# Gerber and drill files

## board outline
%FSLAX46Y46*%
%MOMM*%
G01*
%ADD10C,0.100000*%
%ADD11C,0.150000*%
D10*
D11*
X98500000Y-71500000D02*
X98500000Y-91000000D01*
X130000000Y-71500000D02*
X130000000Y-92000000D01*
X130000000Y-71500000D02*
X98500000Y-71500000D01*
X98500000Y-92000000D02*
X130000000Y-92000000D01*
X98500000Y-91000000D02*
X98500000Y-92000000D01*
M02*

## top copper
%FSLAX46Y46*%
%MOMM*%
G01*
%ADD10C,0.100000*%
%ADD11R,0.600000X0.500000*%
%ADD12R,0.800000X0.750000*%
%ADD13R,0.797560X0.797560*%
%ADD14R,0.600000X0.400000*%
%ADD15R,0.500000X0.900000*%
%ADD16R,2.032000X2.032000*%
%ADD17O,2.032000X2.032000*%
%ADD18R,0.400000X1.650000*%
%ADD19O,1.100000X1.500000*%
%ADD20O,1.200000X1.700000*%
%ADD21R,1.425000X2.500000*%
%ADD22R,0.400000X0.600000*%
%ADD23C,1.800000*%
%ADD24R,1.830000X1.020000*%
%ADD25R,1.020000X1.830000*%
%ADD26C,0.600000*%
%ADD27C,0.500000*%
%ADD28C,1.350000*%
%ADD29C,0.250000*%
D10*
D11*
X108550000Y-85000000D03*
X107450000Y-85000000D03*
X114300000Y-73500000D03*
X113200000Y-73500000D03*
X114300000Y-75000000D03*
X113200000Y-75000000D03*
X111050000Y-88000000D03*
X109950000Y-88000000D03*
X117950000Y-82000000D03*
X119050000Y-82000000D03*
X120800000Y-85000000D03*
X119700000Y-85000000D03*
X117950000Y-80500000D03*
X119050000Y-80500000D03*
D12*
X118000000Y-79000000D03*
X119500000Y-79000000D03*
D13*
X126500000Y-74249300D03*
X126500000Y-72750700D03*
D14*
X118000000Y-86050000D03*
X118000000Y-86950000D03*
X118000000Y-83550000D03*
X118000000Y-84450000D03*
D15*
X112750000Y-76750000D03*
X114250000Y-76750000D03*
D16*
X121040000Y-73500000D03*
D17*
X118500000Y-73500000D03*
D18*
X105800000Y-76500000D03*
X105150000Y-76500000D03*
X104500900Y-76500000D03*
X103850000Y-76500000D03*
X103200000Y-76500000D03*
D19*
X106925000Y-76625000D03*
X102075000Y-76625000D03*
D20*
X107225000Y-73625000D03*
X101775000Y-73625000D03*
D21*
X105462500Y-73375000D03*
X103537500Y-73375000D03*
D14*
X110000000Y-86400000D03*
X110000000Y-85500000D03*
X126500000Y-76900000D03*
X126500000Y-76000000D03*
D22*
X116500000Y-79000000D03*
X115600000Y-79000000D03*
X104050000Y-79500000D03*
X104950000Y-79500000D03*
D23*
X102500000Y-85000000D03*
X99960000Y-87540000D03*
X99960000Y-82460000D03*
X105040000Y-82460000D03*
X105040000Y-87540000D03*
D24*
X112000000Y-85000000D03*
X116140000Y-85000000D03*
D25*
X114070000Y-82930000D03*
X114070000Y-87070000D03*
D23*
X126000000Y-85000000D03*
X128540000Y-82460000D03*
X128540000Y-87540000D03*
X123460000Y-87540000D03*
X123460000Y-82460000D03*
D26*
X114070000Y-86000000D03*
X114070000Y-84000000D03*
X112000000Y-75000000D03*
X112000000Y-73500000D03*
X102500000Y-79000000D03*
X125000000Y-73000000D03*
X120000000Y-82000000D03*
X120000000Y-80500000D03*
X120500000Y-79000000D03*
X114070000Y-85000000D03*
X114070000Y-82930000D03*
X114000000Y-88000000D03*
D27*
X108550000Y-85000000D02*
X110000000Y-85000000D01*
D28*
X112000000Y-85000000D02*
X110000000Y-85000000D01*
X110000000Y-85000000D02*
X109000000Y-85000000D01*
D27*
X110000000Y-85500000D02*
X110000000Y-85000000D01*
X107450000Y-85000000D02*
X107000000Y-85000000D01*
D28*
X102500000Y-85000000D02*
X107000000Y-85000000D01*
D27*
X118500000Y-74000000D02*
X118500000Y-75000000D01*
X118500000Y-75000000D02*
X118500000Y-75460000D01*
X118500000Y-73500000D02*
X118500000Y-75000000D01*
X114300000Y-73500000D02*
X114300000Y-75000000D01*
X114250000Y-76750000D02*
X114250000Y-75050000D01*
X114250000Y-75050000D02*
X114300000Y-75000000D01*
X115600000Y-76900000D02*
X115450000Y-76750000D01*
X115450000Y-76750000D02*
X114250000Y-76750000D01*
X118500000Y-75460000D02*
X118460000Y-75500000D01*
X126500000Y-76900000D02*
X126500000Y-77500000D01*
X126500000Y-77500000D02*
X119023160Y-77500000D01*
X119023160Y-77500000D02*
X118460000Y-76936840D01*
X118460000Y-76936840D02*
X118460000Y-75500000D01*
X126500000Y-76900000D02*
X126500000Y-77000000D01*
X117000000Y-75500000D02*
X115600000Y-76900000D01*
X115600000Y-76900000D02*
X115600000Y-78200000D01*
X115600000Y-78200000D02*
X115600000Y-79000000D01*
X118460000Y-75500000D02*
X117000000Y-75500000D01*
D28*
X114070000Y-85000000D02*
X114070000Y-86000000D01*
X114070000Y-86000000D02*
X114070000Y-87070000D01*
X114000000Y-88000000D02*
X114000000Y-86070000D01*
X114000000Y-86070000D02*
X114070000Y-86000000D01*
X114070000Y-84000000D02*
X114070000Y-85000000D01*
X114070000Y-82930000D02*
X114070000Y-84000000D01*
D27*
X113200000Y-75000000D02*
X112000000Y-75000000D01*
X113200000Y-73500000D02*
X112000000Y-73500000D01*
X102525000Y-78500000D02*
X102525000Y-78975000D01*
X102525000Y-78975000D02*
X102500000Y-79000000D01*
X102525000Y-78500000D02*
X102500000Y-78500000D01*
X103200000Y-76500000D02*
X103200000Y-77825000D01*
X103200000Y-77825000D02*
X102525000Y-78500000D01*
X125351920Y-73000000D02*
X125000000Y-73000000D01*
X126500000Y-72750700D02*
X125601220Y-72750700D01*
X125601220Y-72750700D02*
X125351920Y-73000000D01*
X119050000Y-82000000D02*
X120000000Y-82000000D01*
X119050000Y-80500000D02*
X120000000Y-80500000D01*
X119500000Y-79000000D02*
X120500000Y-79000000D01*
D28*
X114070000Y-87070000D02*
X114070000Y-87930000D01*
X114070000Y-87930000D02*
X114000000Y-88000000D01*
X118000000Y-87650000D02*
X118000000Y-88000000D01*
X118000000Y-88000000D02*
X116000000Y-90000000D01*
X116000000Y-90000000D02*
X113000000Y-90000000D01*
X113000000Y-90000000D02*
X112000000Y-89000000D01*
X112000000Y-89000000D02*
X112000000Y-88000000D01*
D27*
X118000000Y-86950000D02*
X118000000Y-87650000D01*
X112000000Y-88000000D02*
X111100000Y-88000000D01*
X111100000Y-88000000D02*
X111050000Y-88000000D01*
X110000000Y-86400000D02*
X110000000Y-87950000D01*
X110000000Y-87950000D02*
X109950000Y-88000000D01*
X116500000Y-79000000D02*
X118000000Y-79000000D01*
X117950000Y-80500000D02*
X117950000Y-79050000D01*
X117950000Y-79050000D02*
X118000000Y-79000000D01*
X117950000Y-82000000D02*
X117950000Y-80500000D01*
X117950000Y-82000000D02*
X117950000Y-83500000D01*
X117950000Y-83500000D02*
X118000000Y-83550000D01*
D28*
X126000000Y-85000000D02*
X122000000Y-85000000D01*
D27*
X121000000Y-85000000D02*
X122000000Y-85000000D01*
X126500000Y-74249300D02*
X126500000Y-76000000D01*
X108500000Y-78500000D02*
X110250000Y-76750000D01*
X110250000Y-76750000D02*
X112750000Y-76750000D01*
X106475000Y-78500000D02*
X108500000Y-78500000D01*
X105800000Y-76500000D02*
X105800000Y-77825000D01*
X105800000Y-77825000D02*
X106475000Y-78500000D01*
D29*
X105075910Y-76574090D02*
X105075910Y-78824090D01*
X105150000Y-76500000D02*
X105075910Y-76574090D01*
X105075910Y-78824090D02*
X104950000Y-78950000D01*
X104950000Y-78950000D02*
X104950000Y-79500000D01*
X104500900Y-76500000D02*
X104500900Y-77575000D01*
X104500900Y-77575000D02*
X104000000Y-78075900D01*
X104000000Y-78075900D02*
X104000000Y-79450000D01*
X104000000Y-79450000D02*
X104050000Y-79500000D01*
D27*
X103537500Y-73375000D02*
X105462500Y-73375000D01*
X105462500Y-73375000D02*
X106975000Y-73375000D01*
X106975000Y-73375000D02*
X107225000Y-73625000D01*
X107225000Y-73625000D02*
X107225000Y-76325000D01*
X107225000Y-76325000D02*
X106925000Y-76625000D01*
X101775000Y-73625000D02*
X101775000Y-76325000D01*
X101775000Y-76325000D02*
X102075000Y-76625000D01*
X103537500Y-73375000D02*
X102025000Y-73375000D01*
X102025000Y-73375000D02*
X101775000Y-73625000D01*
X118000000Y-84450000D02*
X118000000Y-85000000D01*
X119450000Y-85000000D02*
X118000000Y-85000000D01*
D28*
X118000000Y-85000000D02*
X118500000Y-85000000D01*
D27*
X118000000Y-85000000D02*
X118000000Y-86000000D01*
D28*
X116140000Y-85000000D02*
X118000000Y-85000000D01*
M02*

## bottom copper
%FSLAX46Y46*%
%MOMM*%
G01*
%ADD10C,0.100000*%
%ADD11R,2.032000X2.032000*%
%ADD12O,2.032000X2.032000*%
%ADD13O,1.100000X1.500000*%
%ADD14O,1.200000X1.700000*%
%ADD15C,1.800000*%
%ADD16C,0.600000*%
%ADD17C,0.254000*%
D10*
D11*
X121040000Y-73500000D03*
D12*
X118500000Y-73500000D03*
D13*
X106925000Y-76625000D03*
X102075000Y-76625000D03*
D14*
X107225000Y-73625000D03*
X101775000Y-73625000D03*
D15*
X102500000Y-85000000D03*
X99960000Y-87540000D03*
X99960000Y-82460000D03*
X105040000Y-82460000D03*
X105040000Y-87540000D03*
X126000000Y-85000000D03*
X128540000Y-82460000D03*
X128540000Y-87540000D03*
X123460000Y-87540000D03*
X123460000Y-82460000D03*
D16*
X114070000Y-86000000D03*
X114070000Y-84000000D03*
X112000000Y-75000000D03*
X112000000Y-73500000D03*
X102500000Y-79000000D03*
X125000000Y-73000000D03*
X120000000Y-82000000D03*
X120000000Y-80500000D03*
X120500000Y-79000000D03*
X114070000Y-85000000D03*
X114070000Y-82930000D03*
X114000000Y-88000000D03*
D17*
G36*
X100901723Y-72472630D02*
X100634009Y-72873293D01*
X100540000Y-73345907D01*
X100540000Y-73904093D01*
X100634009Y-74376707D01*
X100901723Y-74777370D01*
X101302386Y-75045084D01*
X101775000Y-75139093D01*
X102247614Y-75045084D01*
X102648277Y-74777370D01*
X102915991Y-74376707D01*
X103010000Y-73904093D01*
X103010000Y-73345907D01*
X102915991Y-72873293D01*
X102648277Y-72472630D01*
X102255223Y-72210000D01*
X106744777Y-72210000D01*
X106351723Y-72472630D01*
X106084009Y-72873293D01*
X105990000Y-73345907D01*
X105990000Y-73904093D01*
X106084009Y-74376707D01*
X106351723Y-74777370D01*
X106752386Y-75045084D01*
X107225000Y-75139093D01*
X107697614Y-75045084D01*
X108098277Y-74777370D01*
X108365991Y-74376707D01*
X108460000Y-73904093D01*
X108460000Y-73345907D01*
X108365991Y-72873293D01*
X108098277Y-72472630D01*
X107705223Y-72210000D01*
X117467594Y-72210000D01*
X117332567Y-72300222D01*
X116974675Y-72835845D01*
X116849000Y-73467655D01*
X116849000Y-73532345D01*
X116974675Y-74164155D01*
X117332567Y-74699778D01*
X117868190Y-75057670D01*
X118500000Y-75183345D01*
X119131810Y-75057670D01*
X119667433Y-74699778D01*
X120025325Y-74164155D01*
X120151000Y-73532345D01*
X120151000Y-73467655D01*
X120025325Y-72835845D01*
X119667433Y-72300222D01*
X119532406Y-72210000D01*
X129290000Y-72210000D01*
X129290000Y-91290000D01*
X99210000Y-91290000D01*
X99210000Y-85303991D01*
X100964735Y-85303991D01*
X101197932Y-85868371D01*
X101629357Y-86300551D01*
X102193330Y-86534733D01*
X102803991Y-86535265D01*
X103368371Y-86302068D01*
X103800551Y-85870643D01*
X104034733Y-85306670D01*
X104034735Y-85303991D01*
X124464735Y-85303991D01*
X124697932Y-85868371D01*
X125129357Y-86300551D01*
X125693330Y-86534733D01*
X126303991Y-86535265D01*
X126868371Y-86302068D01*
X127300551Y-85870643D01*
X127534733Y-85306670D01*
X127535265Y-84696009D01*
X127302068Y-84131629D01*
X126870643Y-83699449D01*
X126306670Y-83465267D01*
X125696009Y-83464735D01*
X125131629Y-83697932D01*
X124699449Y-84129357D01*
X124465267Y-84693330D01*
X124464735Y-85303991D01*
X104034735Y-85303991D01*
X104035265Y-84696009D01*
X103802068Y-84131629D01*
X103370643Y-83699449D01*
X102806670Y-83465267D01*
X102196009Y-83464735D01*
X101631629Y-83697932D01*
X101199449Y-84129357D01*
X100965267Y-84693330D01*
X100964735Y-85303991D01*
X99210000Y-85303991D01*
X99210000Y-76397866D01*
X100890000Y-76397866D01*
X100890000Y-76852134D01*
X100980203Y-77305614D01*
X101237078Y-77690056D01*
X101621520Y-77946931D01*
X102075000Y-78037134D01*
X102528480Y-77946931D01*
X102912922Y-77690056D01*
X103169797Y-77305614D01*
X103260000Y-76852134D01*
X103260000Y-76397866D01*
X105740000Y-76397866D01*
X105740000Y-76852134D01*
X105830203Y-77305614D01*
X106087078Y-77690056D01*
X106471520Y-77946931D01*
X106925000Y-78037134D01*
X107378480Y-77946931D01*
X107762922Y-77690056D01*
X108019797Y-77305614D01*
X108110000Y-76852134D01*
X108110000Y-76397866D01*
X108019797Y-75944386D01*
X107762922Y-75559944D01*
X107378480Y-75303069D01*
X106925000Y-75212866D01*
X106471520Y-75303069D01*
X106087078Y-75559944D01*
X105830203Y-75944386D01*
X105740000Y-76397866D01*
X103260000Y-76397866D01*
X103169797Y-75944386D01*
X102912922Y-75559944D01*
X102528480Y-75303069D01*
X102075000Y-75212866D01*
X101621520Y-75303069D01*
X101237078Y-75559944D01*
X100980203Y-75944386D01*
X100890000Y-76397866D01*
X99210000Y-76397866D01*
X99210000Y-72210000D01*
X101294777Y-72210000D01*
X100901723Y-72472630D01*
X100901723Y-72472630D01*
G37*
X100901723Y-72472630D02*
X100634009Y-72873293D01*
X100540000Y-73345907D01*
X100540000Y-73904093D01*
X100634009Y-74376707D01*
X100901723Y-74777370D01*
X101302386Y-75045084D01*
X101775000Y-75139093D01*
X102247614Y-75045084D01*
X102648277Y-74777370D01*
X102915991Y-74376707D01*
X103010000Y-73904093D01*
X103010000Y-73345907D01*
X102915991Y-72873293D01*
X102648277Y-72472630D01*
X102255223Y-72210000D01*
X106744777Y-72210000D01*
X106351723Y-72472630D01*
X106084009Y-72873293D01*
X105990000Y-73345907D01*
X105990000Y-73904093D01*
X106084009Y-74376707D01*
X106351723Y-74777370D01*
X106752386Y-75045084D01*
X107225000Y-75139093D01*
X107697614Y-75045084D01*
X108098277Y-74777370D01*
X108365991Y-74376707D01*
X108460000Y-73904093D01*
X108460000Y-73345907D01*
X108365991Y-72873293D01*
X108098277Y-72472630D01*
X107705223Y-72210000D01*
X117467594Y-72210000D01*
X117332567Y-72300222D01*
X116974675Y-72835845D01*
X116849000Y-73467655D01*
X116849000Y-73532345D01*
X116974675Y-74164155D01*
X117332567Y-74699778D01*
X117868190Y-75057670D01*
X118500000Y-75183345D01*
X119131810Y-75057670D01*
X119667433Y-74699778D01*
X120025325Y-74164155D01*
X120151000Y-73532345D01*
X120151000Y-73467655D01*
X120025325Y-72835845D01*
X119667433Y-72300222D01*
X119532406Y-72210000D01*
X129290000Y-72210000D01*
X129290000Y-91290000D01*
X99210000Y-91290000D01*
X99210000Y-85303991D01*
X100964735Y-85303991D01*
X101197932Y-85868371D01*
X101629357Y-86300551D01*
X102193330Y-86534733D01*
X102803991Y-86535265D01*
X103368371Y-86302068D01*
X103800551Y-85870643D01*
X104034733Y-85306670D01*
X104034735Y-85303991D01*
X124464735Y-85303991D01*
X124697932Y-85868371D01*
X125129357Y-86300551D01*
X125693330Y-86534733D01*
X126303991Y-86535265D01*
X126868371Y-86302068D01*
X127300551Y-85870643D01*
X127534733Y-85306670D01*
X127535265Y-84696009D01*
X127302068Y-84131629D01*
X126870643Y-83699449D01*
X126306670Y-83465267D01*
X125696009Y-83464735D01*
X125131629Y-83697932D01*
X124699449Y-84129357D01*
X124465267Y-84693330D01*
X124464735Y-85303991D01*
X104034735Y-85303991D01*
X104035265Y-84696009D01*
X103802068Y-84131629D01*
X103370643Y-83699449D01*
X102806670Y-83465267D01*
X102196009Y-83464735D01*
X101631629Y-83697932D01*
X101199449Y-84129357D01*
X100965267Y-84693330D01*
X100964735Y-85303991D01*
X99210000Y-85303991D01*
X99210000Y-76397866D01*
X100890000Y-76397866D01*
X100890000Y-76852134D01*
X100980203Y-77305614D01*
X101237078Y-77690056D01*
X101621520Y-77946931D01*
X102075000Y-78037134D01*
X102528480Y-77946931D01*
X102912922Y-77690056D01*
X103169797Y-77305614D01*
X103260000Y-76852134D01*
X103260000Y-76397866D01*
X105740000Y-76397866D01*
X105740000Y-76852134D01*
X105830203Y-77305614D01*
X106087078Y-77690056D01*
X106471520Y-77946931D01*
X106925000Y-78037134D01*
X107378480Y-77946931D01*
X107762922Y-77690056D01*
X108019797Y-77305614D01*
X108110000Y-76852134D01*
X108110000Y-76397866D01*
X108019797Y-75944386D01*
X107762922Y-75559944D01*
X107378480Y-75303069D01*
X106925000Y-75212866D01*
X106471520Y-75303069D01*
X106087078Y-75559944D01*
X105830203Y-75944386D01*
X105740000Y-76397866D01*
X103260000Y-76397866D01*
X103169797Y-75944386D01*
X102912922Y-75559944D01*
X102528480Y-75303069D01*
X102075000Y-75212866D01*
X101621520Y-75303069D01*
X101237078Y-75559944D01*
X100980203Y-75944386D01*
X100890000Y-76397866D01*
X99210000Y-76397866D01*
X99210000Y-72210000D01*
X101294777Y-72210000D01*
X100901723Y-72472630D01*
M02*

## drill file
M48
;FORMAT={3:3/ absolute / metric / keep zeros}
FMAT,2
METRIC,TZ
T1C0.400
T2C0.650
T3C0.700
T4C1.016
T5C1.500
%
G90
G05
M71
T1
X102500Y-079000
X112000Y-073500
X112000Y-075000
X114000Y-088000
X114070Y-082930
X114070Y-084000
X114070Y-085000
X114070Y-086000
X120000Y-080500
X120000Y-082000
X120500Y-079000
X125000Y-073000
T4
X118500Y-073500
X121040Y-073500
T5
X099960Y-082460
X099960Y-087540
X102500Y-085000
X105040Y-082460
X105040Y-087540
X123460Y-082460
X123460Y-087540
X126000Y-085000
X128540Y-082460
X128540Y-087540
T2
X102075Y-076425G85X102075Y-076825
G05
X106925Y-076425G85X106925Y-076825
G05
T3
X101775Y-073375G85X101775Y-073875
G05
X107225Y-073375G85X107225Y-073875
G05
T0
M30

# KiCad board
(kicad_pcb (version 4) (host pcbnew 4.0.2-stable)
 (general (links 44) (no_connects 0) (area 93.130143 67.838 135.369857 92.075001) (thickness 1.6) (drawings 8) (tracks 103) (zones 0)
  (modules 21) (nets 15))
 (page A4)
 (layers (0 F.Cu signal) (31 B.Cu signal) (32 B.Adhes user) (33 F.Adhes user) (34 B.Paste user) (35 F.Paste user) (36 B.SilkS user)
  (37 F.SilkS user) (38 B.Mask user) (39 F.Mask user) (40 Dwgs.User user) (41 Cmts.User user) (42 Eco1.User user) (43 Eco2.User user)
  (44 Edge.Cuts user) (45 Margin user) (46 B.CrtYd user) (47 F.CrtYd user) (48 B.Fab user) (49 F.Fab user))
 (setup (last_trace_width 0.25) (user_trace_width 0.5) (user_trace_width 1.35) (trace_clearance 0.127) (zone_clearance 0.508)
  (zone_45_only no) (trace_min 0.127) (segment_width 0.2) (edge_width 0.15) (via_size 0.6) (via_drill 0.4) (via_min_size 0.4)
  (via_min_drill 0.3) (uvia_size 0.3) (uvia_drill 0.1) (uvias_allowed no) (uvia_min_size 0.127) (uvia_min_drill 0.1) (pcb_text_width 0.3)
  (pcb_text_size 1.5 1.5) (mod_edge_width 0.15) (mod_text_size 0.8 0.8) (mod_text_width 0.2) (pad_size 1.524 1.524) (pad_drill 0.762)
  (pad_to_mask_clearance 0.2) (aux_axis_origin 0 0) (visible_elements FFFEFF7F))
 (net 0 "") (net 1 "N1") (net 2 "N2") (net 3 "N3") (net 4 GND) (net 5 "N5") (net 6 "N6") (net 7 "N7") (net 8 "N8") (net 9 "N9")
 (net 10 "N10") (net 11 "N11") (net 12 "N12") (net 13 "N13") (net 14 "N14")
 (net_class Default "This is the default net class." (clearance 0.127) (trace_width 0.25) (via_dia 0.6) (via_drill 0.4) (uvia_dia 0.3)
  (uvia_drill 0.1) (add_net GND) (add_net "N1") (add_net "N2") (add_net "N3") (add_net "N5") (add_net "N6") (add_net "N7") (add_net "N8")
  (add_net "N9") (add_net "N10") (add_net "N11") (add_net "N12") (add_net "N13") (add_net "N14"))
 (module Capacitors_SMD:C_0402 (layer F.Cu) (at 108 85 180)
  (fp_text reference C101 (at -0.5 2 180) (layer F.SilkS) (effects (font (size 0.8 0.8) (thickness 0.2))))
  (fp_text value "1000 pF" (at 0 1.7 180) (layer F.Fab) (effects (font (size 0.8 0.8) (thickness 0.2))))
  (pad 1 smd rect (at -0.55 0 180) (size 0.6 0.5) (layers F.Cu F.Paste F.Mask) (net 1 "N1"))
  (pad 2 smd rect (at 0.55 0 180) (size 0.6 0.5) (layers F.Cu F.Paste F.Mask) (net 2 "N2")))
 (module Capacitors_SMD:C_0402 (layer F.Cu) (at 113.75 73.5 180)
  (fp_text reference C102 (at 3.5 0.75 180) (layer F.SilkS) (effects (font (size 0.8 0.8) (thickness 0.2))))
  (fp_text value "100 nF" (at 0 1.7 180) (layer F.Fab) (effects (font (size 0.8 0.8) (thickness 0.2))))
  (pad 1 smd rect (at -0.55 0 180) (size 0.6 0.5) (layers F.Cu F.Paste F.Mask) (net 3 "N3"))
  (pad 2 smd rect (at 0.55 0 180) (size 0.6 0.5) (layers F.Cu F.Paste F.Mask) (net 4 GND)))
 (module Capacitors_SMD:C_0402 (layer F.Cu) (at 113.75 75 180)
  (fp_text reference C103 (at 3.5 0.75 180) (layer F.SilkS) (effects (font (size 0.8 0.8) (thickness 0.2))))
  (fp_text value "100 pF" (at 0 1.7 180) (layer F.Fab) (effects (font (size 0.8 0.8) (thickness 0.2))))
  (pad 1 smd rect (at -0.55 0 180) (size 0.6 0.5) (layers F.Cu F.Paste F.Mask) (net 3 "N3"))
  (pad 2 smd rect (at 0.55 0 180) (size 0.6 0.5) (layers F.Cu F.Paste F.Mask) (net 4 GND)))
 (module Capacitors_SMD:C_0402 (layer F.Cu) (at 110.5 88 180)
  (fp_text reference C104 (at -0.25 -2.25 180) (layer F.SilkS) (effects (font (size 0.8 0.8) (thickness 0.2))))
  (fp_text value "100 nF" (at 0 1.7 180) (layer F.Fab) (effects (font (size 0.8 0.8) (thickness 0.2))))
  (pad 1 smd rect (at -0.55 0 180) (size 0.6 0.5) (layers F.Cu F.Paste F.Mask) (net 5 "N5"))
  (pad 2 smd rect (at 0.55 0 180) (size 0.6 0.5) (layers F.Cu F.Paste F.Mask) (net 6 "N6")))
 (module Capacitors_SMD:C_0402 (layer F.Cu) (at 118.5 82)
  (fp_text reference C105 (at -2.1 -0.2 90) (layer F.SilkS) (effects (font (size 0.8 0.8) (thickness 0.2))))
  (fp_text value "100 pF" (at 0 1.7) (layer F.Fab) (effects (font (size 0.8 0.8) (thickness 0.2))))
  (pad 1 smd rect (at -0.55 0) (size 0.6 0.5) (layers F.Cu F.Paste F.Mask) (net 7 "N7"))
  (pad 2 smd rect (at 0.55 0) (size 0.6 0.5) (layers F.Cu F.Paste F.Mask) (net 4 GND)))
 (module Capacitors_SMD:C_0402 (layer F.Cu) (at 120.25 85 180)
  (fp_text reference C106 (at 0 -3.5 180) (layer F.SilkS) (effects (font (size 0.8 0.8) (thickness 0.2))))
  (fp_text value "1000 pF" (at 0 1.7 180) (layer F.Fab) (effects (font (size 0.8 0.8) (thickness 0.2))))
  (pad 1 smd rect (at -0.55 0 180) (size 0.6 0.5) (layers F.Cu F.Paste F.Mask) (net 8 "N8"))
  (pad 2 smd rect (at 0.55 0 180) (size 0.6 0.5) (layers F.Cu F.Paste F.Mask) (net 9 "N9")))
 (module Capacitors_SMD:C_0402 (layer F.Cu) (at 118.5 80.5)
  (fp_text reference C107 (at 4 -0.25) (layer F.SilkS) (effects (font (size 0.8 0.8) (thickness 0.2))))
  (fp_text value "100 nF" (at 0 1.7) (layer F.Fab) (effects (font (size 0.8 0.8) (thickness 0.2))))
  (pad 1 smd rect (at -0.55 0) (size 0.6 0.5) (layers F.Cu F.Paste F.Mask) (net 7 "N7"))
  (pad 2 smd rect (at 0.55 0) (size 0.6 0.5) (layers F.Cu F.Paste F.Mask) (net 4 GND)))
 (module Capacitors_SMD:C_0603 (layer F.Cu) (at 118.75 79)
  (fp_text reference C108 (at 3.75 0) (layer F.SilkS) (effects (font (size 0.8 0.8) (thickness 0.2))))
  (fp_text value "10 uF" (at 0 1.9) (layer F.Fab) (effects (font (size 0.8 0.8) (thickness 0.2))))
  (pad 1 smd rect (at -0.75 0) (size 0.8 0.75) (layers F.Cu F.Paste F.Mask) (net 7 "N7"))
  (pad 2 smd rect (at 0.75 0) (size 0.8 0.75) (layers F.Cu F.Paste F.Mask) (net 4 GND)))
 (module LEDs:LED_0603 (layer F.Cu) (at 126.5 73.5 270)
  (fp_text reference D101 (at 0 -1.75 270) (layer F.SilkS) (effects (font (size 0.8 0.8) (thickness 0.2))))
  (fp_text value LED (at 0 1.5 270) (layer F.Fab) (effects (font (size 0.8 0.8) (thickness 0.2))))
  (pad 2 smd rect (at 0.7493 0 90) (size 0.79756 0.79756) (layers F.Cu F.Paste F.Mask) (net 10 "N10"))
  (pad 1 smd rect (at -0.7493 0 90) (size 0.79756 0.79756) (layers F.Cu F.Paste F.Mask) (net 4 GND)))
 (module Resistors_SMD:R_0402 (layer F.Cu) (at 118 86.5 270)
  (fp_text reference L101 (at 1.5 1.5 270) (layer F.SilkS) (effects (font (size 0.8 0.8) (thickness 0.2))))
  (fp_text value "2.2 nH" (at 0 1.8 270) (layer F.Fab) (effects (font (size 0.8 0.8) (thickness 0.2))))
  (pad 1 smd rect (at -0.45 0 270) (size 0.4 0.6) (layers F.Cu F.Paste F.Mask) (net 9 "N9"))
  (pad 2 smd rect (at 0.45 0 270) (size 0.4 0.6) (layers F.Cu F.Paste F.Mask) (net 5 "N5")))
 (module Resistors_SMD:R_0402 (layer F.Cu) (at 118 84 270)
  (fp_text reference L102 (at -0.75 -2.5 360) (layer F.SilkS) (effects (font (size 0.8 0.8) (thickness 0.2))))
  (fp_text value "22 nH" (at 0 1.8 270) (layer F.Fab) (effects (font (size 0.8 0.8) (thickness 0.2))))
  (pad 1 smd rect (at -0.45 0 270) (size 0.4 0.6) (layers F.Cu F.Paste F.Mask) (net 7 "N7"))
  (pad 2 smd rect (at 0.45 0 270) (size 0.4 0.6) (layers F.Cu F.Paste F.Mask) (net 9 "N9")))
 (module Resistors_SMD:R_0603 (layer F.Cu) (at 113.5 76.75)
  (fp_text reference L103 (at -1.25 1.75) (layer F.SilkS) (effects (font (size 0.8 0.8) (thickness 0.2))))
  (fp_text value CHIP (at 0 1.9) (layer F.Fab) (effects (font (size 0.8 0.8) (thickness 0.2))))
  (pad 1 smd rect (at -0.75 0) (size 0.5 0.9) (layers F.Cu F.Paste F.Mask) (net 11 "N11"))
  (pad 2 smd rect (at 0.75 0) (size 0.5 0.9) (layers F.Cu F.Paste F.Mask) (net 3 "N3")))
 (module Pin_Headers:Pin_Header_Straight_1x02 (layer F.Cu) (at 121.04 73.5 270)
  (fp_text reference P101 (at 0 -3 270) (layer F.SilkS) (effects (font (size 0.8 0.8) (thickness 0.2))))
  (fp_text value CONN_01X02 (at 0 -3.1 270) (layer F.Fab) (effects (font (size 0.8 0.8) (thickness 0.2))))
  (pad 1 thru_hole rect (at 0 0 270) (size 2.032 2.032) (drill 1.016) (layers *.Cu *.Mask F.SilkS) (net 4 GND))
  (pad 2 thru_hole oval (at 0 2.54 270) (size 2.032 2.032) (drill 1.016) (layers *.Cu *.Mask F.SilkS) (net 3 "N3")))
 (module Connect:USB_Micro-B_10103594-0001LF (layer F.Cu) (at 104.5 75 180)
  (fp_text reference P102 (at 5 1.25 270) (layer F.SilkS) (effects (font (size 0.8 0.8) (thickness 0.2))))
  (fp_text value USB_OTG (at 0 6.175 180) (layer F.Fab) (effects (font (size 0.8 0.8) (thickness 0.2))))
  (pad 1 smd rect (at -1.3 -1.5 270) (size 1.65 0.4) (layers F.Cu F.Paste F.Mask) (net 11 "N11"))
  (pad 2 smd rect (at -0.65 -1.5 270) (size 1.65 0.4) (layers F.Cu F.Paste F.Mask) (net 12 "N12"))
  (pad 3 smd rect (at -0.0009 -1.5 270) (size 1.65 0.4) (layers F.Cu F.Paste F.Mask) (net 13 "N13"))
  (pad 4 smd rect (at 0.65 -1.5 270) (size 1.65 0.4) (layers F.Cu F.Paste F.Mask))
  (pad 5 smd rect (at 1.3 -1.5 270) (size 1.65 0.4) (layers F.Cu F.Paste F.Mask) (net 4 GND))
  (pad 6 thru_hole oval (at -2.425 -1.625 270) (size 1.5 1.1) (drill oval 1.05 0.65) (layers *.Cu *.Mask F.SilkS) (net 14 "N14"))
  (pad 6 thru_hole oval (at 2.425 -1.625 270) (size 1.5 1.1) (drill oval 1.05 0.65) (layers *.Cu *.Mask F.SilkS) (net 14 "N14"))
  (pad 6 thru_hole oval (at -2.725 1.375 270) (size 1.7 1.2) (drill oval 1.2 0.7) (layers *.Cu *.Mask F.SilkS) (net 14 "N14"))
  (pad 6 thru_hole oval (at 2.725 1.375 270) (size 1.7 1.2) (drill oval 1.2 0.7) (layers *.Cu *.Mask F.SilkS) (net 14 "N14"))
  (pad 6 smd rect (at -0.9625 1.625 270) (size 2.5 1.425) (layers F.Cu F.Paste F.Mask) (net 14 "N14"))
  (pad 6 smd rect (at 0.9625 1.625 270) (size 2.5 1.425) (layers F.Cu F.Paste F.Mask) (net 14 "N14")))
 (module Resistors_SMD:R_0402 (layer F.Cu) (at 110 85.95 90)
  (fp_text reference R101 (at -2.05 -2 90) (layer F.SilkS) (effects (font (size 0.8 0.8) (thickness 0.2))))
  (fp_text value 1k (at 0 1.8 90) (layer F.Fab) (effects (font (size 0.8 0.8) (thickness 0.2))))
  (pad 1 smd rect (at -0.45 0 90) (size 0.4 0.6) (layers F.Cu F.Paste F.Mask) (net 6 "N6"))
  (pad 2 smd rect (at 0.45 0 90) (size 0.4 0.6) (layers F.Cu F.Paste F.Mask) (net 1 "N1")))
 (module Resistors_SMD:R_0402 (layer F.Cu) (at 126.5 76.45 90)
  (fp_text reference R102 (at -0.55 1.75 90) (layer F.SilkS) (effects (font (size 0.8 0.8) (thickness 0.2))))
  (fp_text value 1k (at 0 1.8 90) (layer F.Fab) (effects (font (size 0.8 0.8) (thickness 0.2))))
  (pad 1 smd rect (at -0.45 0 90) (size 0.4 0.6) (layers F.Cu F.Paste F.Mask) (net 3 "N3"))
  (pad 2 smd rect (at 0.45 0 90) (size 0.4 0.6) (layers F.Cu F.Paste F.Mask) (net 10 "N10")))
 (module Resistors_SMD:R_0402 (layer F.Cu) (at 116.05 79 180)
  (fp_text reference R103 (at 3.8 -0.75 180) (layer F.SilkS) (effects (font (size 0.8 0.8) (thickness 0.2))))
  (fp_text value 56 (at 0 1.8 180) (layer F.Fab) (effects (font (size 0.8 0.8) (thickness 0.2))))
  (pad 1 smd rect (at -0.45 0 180) (size 0.4 0.6) (layers F.Cu F.Paste F.Mask) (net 7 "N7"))
  (pad 2 smd rect (at 0.45 0 180) (size 0.4 0.6) (layers F.Cu F.Paste F.Mask) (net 3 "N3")))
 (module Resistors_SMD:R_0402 (layer F.Cu) (at 104.5 79.5)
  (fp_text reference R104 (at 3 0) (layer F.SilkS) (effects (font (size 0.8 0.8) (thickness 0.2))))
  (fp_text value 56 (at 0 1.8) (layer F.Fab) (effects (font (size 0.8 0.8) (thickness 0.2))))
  (pad 1 smd rect (at -0.45 0) (size 0.4 0.6) (layers F.Cu F.Paste F.Mask) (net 13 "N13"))
  (pad 2 smd rect (at 0.45 0) (size 0.4 0.6) (layers F.Cu F.Paste F.Mask) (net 12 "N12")))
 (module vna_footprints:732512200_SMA (layer F.Cu) (at 102.5 85)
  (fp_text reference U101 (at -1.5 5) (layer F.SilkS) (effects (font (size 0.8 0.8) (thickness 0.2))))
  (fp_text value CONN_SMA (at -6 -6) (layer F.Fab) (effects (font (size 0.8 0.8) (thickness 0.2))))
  (pad 1 thru_hole circle (at 0 0) (size 1.8 1.8) (drill 1.5) (layers *.Cu *.Mask F.SilkS) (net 2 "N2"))
  (pad 2 thru_hole circle (at -2.54 2.54) (size 1.8 1.8) (drill 1.5) (layers *.Cu *.Mask F.SilkS) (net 4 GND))
  (pad 3 thru_hole circle (at -2.54 -2.54) (size 1.8 1.8) (drill 1.5) (layers *.Cu *.Mask F.SilkS) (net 4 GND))
  (pad 4 thru_hole circle (at 2.54 -2.54) (size 1.8 1.8) (drill 1.5) (layers *.Cu *.Mask F.SilkS) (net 4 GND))
  (pad 5 thru_hole circle (at 2.54 2.54) (size 1.8 1.8) (drill 1.5) (layers *.Cu *.Mask F.SilkS) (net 4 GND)))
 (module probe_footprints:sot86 (layer F.Cu) (at 114.07 85)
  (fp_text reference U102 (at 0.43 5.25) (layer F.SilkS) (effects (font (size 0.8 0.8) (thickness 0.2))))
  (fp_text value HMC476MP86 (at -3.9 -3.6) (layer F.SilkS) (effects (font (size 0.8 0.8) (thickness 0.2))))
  (pad 1 smd rect (at -2.07 0 180) (size 1.83 1.02) (layers F.Cu F.Paste F.Mask) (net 1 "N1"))
  (pad 3 smd rect (at 2.07 0 180) (size 1.83 1.02) (layers F.Cu F.Paste F.Mask) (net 9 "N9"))
  (pad 4 smd rect (at 0 -2.07 270) (size 1.83 1.02) (layers F.Cu F.Paste F.Mask) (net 4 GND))
  (pad 2 smd rect (at 0 2.07 270) (size 1.83 1.02) (layers F.Cu F.Paste F.Mask) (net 4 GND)))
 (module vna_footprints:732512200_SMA (layer F.Cu) (at 126 85 180)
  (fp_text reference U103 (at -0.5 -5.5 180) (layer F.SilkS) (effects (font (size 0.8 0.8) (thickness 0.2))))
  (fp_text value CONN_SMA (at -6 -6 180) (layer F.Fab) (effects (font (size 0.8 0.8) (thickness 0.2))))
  (pad 1 thru_hole circle (at 0 0 180) (size 1.8 1.8) (drill 1.5) (layers *.Cu *.Mask F.SilkS) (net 8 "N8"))
  (pad 2 thru_hole circle (at -2.54 2.54 180) (size 1.8 1.8) (drill 1.5) (layers *.Cu *.Mask F.SilkS) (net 4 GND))
  (pad 3 thru_hole circle (at -2.54 -2.54 180) (size 1.8 1.8) (drill 1.5) (layers *.Cu *.Mask F.SilkS) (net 4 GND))
  (pad 4 thru_hole circle (at 2.54 -2.54 180) (size 1.8 1.8) (drill 1.5) (layers *.Cu *.Mask F.SilkS) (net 4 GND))
  (pad 5 thru_hole circle (at 2.54 2.54 180) (size 1.8 1.8) (drill 1.5) (layers *.Cu *.Mask F.SilkS) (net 4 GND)))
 (gr_line (start 98.5 71.5) (end 98.5 91) (layer Edge.Cuts) (width 0.15))
 (gr_line (start 130 71.5) (end 130 92) (layer Edge.Cuts) (width 0.15))
 (gr_line (start 130 71.5) (end 98.5 71.5) (layer Edge.Cuts) (width 0.15))
 (gr_line (start 98.5 92) (end 130 92) (layer Edge.Cuts) (width 0.15))
 (gr_line (start 98.5 91) (end 98.5 92) (layer Edge.Cuts) (width 0.15))
 (segment (start 108.55 85) (end 110 85) (width 0.5) (layer F.Cu) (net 1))
 (segment (start 112 85) (end 110 85) (width 1.35) (layer F.Cu) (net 1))
 (segment (start 110 85) (end 109 85) (width 1.35) (layer F.Cu) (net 1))
 (segment (start 110 85.5) (end 110 85) (width 0.5) (layer F.Cu) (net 1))
 (segment (start 107.45 85) (end 107 85) (width 0.5) (layer F.Cu) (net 2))
 (segment (start 102.5 85) (end 107 85) (width 1.35) (layer F.Cu) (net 2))
 (segment (start 118.5 74) (end 118.5 75) (width 0.5) (layer F.Cu) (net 3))
 (segment (start 118.5 75) (end 118.5 75.46) (width 0.5) (layer F.Cu) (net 3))
 (segment (start 118.5 73.5) (end 118.5 75) (width 0.5) (layer F.Cu) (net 3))
 (segment (start 114.3 73.5) (end 114.3 75) (width 0.5) (layer F.Cu) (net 3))
 (segment (start 114.25 76.75) (end 114.25 75.05) (width 0.5) (layer F.Cu) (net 3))
 (segment (start 114.25 75.05) (end 114.3 75) (width 0.5) (layer F.Cu) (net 3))
 (segment (start 115.6 76.9) (end 115.45 76.75) (width 0.5) (layer F.Cu) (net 3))
 (segment (start 115.45 76.75) (end 114.25 76.75) (width 0.5) (layer F.Cu) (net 3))
 (segment (start 118.5 75.46) (end 118.46 75.5) (width 0.5) (layer F.Cu) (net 3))
 (segment (start 126.5 76.9) (end 126.5 77.5) (width 0.5) (layer F.Cu) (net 3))
 (segment (start 126.5 77.5) (end 119.02316 77.5) (width 0.5) (layer F.Cu) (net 3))
 (segment (start 119.02316 77.5) (end 118.46 76.93684) (width 0.5) (layer F.Cu) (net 3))
 (segment (start 118.46 76.93684) (end 118.46 75.5) (width 0.5) (layer F.Cu) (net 3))
 (segment (start 126.5 76.9) (end 126.5 77) (width 0.5) (layer F.Cu) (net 3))
 (segment (start 117 75.5) (end 115.6 76.9) (width 0.5) (layer F.Cu) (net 3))
 (segment (start 115.6 76.9) (end 115.6 78.2) (width 0.5) (layer F.Cu) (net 3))
 (segment (start 115.6 78.2) (end 115.6 79) (width 0.5) (layer F.Cu) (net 3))
 (segment (start 118.46 75.5) (end 117 75.5) (width 0.5) (layer F.Cu) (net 3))
 (segment (start 114.07 85) (end 114.07 86) (width 1.35) (layer F.Cu) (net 4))
 (segment (start 114.07 86) (end 114.07 87.07) (width 1.35) (layer F.Cu) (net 4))
 (segment (start 114 88) (end 114 86.07) (width 1.35) (layer F.Cu) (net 4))
 (segment (start 114 86.07) (end 114.07 86) (width 1.35) (layer F.Cu) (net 4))
 (via (at 114.07 86) (size 0.6) (drill 0.4) (layers F.Cu B.Cu) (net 4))
 (segment (start 114.07 84) (end 114.07 85) (width 1.35) (layer F.Cu) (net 4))
 (segment (start 114.07 82.93) (end 114.07 84) (width 1.35) (layer F.Cu) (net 4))
 (via (at 114.07 84) (size 0.6) (drill 0.4) (layers F.Cu B.Cu) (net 4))
 (via (at 112 75) (size 0.6) (drill 0.4) (layers F.Cu B.Cu) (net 4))
 (segment (start 113.2 75) (end 112 75) (width 0.5) (layer F.Cu) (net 4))
 (via (at 112 73.5) (size 0.6) (drill 0.4) (layers F.Cu B.Cu) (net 4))
 (segment (start 113.2 73.5) (end 112 73.5) (width 0.5) (layer F.Cu) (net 4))
 (segment (start 102.525 78.5) (end 102.525 78.975) (width 0.5) (layer F.Cu) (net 4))
 (segment (start 102.525 78.975) (end 102.5 79) (width 0.5) (layer F.Cu) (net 4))
 (via (at 102.5 79) (size 0.6) (drill 0.4) (layers F.Cu B.Cu) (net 4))
 (segment (start 102.525 78.5) (end 102.5 78.5) (width 0.5) (layer F.Cu) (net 4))
 (segment (start 103.2 76.5) (end 103.2 77.825) (width 0.5) (layer F.Cu) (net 4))
 (segment (start 103.2 77.825) (end 102.525 78.5) (width 0.5) (layer F.Cu) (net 4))
 (segment (start 125.35192 73) (end 125 73) (width 0.5) (layer F.Cu) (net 4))
 (via (at 125 73) (size 0.6) (drill 0.4) (layers F.Cu B.Cu) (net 4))
 (segment (start 126.5 72.7507) (end 125.60122 72.7507) (width 0.5) (layer F.Cu) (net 4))
 (segment (start 125.60122 72.7507) (end 125.35192 73) (width 0.5) (layer F.Cu) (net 4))
 (segment (start 119.05 82) (end 120 82) (width 0.5) (layer F.Cu) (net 4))
 (via (at 120 82) (size 0.6) (drill 0.4) (layers F.Cu B.Cu) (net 4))
 (via (at 120 80.5) (size 0.6) (drill 0.4) (layers F.Cu B.Cu) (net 4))
 (segment (start 119.05 80.5) (end 120 80.5) (width 0.5) (layer F.Cu) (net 4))
 (via (at 120.5 79) (size 0.6) (drill 0.4) (layers F.Cu B.Cu) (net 4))
 (segment (start 119.5 79) (end 120.5 79) (width 0.5) (layer F.Cu) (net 4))
 (via (at 114.07 85) (size 0.6) (drill 0.4) (layers F.Cu B.Cu) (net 4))
 (via (at 114.07 82.93) (size 0.6) (drill 0.4) (layers F.Cu B.Cu) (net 4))
 (segment (start 114.07 87.07) (end 114.07 87.93) (width 1.35) (layer F.Cu) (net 4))
 (segment (start 114.07 87.93) (end 114 88) (width 1.35) (layer F.Cu) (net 4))
 (via (at 114 88) (size 0.6) (drill 0.4) (layers F.Cu B.Cu) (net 4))
 (segment (start 118 87.65) (end 118 88) (width 1.35) (layer F.Cu) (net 5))
 (segment (start 118 88) (end 116 90) (width 1.35) (layer F.Cu) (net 5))
 (segment (start 116 90) (end 113 90) (width 1.35) (layer F.Cu) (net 5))
 (segment (start 113 90) (end 112 89) (width 1.35) (layer F.Cu) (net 5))
 (segment (start 112 89) (end 112 88) (width 1.35) (layer F.Cu) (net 5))
 (segment (start 118 86.95) (end 118 87.65) (width 0.5) (layer F.Cu) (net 5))
 (segment (start 112 88) (end 111.1 88) (width 0.5) (layer F.Cu) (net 5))
 (segment (start 111.1 88) (end 111.05 88) (width 0.5) (layer F.Cu) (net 5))
 (segment (start 110 86.4) (end 110 87.95) (width 0.5) (layer F.Cu) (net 6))
 (segment (start 110 87.95) (end 109.95 88) (width 0.5) (layer F.Cu) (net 6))
 (segment (start 116.5 79) (end 118 79) (width 0.5) (layer F.Cu) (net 7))
 (segment (start 117.95 80.5) (end 117.95 79.05) (width 0.5) (layer F.Cu) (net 7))
 (segment (start 117.95 79.05) (end 118 79) (width 0.5) (layer F.Cu) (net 7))
 (segment (start 117.95 82) (end 117.95 80.5) (width 0.5) (layer F.Cu) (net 7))
 (segment (start 117.95 82) (end 117.95 83.5) (width 0.5) (layer F.Cu) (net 7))
 (segment (start 117.95 83.5) (end 118 83.55) (width 0.5) (layer F.Cu) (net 7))
 (segment (start 126 85) (end 122 85) (width 1.35) (layer F.Cu) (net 8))
 (segment (start 121 85) (end 122 85) (width 0.5) (layer F.Cu) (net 8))
 (segment (start 126.5 74.2493) (end 126.5 76) (width 0.5) (layer F.Cu) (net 10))
 (segment (start 108.5 78.5) (end 110.25 76.75) (width 0.5) (layer F.Cu) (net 11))
 (segment (start 110.25 76.75) (end 112.75 76.75) (width 0.5) (layer F.Cu) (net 11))
 (segment (start 106.475 78.5) (end 108.5 78.5) (width 0.5) (layer F.Cu) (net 11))
 (segment (start 105.8 76.5) (end 105.8 77.825) (width 0.5) (layer F.Cu) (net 11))
 (segment (start 105.8 77.825) (end 106.475 78.5) (width 0.5) (layer F.Cu) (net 11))
 (segment (start 105.07591 76.57409) (end 105.07591 78.82409) (width 0.25) (layer F.Cu) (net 12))
 (segment (start 105.15 76.5) (end 105.07591 76.57409) (width 0.25) (layer F.Cu) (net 12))
 (segment (start 105.07591 78.82409) (end 104.95 78.95) (width 0.25) (layer F.Cu) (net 12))
 (segment (start 104.95 78.95) (end 104.95 79.5) (width 0.25) (layer F.Cu) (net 12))
 (segment (start 104.5009 76.5) (end 104.5009 77.575) (width 0.25) (layer F.Cu) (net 13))
 (segment (start 104.5009 77.575) (end 104 78.0759) (width 0.25) (layer F.Cu) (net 13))
 (segment (start 104 78.0759) (end 104 79.45) (width 0.25) (layer F.Cu) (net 13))
 (segment (start 104 79.45) (end 104.05 79.5) (width 0.25) (layer F.Cu) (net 13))
 (segment (start 103.5375 73.375) (end 105.4625 73.375) (width 0.5) (layer F.Cu) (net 14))
 (segment (start 105.4625 73.375) (end 106.975 73.375) (width 0.5) (layer F.Cu) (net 14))
 (segment (start 106.975 73.375) (end 107.225 73.625) (width 0.5) (layer F.Cu) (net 14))
 (segment (start 107.225 73.625) (end 107.225 76.325) (width 0.5) (layer F.Cu) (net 14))
 (segment (start 107.225 76.325) (end 106.925 76.625) (width 0.5) (layer F.Cu) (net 14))
 (segment (start 101.775 73.625) (end 101.775 76.325) (width 0.5) (layer F.Cu) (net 14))
 (segment (start 101.775 76.325) (end 102.075 76.625) (width 0.5) (layer F.Cu) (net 14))
 (segment (start 103.5375 73.375) (end 102.025 73.375) (width 0.5) (layer F.Cu) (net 14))
 (segment (start 102.025 73.375) (end 101.775 73.625) (width 0.5) (layer F.Cu) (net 14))
 (segment (start 118 84.45) (end 118 85) (width 0.5) (layer F.Cu) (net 9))
 (segment (start 119.45 85) (end 118 85) (width 0.5) (layer F.Cu) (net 9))
 (segment (start 118 85) (end 118.5 85) (width 1.35) (layer F.Cu) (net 9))
 (segment (start 118 85) (end 118 86) (width 0.5) (layer F.Cu) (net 9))
 (segment (start 116.14 85) (end 118 85) (width 1.35) (layer F.Cu) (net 9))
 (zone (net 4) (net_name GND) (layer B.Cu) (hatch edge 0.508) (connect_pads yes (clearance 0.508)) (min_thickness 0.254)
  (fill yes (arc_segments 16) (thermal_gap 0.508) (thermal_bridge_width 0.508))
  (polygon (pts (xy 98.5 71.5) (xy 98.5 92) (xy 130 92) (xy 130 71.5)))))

